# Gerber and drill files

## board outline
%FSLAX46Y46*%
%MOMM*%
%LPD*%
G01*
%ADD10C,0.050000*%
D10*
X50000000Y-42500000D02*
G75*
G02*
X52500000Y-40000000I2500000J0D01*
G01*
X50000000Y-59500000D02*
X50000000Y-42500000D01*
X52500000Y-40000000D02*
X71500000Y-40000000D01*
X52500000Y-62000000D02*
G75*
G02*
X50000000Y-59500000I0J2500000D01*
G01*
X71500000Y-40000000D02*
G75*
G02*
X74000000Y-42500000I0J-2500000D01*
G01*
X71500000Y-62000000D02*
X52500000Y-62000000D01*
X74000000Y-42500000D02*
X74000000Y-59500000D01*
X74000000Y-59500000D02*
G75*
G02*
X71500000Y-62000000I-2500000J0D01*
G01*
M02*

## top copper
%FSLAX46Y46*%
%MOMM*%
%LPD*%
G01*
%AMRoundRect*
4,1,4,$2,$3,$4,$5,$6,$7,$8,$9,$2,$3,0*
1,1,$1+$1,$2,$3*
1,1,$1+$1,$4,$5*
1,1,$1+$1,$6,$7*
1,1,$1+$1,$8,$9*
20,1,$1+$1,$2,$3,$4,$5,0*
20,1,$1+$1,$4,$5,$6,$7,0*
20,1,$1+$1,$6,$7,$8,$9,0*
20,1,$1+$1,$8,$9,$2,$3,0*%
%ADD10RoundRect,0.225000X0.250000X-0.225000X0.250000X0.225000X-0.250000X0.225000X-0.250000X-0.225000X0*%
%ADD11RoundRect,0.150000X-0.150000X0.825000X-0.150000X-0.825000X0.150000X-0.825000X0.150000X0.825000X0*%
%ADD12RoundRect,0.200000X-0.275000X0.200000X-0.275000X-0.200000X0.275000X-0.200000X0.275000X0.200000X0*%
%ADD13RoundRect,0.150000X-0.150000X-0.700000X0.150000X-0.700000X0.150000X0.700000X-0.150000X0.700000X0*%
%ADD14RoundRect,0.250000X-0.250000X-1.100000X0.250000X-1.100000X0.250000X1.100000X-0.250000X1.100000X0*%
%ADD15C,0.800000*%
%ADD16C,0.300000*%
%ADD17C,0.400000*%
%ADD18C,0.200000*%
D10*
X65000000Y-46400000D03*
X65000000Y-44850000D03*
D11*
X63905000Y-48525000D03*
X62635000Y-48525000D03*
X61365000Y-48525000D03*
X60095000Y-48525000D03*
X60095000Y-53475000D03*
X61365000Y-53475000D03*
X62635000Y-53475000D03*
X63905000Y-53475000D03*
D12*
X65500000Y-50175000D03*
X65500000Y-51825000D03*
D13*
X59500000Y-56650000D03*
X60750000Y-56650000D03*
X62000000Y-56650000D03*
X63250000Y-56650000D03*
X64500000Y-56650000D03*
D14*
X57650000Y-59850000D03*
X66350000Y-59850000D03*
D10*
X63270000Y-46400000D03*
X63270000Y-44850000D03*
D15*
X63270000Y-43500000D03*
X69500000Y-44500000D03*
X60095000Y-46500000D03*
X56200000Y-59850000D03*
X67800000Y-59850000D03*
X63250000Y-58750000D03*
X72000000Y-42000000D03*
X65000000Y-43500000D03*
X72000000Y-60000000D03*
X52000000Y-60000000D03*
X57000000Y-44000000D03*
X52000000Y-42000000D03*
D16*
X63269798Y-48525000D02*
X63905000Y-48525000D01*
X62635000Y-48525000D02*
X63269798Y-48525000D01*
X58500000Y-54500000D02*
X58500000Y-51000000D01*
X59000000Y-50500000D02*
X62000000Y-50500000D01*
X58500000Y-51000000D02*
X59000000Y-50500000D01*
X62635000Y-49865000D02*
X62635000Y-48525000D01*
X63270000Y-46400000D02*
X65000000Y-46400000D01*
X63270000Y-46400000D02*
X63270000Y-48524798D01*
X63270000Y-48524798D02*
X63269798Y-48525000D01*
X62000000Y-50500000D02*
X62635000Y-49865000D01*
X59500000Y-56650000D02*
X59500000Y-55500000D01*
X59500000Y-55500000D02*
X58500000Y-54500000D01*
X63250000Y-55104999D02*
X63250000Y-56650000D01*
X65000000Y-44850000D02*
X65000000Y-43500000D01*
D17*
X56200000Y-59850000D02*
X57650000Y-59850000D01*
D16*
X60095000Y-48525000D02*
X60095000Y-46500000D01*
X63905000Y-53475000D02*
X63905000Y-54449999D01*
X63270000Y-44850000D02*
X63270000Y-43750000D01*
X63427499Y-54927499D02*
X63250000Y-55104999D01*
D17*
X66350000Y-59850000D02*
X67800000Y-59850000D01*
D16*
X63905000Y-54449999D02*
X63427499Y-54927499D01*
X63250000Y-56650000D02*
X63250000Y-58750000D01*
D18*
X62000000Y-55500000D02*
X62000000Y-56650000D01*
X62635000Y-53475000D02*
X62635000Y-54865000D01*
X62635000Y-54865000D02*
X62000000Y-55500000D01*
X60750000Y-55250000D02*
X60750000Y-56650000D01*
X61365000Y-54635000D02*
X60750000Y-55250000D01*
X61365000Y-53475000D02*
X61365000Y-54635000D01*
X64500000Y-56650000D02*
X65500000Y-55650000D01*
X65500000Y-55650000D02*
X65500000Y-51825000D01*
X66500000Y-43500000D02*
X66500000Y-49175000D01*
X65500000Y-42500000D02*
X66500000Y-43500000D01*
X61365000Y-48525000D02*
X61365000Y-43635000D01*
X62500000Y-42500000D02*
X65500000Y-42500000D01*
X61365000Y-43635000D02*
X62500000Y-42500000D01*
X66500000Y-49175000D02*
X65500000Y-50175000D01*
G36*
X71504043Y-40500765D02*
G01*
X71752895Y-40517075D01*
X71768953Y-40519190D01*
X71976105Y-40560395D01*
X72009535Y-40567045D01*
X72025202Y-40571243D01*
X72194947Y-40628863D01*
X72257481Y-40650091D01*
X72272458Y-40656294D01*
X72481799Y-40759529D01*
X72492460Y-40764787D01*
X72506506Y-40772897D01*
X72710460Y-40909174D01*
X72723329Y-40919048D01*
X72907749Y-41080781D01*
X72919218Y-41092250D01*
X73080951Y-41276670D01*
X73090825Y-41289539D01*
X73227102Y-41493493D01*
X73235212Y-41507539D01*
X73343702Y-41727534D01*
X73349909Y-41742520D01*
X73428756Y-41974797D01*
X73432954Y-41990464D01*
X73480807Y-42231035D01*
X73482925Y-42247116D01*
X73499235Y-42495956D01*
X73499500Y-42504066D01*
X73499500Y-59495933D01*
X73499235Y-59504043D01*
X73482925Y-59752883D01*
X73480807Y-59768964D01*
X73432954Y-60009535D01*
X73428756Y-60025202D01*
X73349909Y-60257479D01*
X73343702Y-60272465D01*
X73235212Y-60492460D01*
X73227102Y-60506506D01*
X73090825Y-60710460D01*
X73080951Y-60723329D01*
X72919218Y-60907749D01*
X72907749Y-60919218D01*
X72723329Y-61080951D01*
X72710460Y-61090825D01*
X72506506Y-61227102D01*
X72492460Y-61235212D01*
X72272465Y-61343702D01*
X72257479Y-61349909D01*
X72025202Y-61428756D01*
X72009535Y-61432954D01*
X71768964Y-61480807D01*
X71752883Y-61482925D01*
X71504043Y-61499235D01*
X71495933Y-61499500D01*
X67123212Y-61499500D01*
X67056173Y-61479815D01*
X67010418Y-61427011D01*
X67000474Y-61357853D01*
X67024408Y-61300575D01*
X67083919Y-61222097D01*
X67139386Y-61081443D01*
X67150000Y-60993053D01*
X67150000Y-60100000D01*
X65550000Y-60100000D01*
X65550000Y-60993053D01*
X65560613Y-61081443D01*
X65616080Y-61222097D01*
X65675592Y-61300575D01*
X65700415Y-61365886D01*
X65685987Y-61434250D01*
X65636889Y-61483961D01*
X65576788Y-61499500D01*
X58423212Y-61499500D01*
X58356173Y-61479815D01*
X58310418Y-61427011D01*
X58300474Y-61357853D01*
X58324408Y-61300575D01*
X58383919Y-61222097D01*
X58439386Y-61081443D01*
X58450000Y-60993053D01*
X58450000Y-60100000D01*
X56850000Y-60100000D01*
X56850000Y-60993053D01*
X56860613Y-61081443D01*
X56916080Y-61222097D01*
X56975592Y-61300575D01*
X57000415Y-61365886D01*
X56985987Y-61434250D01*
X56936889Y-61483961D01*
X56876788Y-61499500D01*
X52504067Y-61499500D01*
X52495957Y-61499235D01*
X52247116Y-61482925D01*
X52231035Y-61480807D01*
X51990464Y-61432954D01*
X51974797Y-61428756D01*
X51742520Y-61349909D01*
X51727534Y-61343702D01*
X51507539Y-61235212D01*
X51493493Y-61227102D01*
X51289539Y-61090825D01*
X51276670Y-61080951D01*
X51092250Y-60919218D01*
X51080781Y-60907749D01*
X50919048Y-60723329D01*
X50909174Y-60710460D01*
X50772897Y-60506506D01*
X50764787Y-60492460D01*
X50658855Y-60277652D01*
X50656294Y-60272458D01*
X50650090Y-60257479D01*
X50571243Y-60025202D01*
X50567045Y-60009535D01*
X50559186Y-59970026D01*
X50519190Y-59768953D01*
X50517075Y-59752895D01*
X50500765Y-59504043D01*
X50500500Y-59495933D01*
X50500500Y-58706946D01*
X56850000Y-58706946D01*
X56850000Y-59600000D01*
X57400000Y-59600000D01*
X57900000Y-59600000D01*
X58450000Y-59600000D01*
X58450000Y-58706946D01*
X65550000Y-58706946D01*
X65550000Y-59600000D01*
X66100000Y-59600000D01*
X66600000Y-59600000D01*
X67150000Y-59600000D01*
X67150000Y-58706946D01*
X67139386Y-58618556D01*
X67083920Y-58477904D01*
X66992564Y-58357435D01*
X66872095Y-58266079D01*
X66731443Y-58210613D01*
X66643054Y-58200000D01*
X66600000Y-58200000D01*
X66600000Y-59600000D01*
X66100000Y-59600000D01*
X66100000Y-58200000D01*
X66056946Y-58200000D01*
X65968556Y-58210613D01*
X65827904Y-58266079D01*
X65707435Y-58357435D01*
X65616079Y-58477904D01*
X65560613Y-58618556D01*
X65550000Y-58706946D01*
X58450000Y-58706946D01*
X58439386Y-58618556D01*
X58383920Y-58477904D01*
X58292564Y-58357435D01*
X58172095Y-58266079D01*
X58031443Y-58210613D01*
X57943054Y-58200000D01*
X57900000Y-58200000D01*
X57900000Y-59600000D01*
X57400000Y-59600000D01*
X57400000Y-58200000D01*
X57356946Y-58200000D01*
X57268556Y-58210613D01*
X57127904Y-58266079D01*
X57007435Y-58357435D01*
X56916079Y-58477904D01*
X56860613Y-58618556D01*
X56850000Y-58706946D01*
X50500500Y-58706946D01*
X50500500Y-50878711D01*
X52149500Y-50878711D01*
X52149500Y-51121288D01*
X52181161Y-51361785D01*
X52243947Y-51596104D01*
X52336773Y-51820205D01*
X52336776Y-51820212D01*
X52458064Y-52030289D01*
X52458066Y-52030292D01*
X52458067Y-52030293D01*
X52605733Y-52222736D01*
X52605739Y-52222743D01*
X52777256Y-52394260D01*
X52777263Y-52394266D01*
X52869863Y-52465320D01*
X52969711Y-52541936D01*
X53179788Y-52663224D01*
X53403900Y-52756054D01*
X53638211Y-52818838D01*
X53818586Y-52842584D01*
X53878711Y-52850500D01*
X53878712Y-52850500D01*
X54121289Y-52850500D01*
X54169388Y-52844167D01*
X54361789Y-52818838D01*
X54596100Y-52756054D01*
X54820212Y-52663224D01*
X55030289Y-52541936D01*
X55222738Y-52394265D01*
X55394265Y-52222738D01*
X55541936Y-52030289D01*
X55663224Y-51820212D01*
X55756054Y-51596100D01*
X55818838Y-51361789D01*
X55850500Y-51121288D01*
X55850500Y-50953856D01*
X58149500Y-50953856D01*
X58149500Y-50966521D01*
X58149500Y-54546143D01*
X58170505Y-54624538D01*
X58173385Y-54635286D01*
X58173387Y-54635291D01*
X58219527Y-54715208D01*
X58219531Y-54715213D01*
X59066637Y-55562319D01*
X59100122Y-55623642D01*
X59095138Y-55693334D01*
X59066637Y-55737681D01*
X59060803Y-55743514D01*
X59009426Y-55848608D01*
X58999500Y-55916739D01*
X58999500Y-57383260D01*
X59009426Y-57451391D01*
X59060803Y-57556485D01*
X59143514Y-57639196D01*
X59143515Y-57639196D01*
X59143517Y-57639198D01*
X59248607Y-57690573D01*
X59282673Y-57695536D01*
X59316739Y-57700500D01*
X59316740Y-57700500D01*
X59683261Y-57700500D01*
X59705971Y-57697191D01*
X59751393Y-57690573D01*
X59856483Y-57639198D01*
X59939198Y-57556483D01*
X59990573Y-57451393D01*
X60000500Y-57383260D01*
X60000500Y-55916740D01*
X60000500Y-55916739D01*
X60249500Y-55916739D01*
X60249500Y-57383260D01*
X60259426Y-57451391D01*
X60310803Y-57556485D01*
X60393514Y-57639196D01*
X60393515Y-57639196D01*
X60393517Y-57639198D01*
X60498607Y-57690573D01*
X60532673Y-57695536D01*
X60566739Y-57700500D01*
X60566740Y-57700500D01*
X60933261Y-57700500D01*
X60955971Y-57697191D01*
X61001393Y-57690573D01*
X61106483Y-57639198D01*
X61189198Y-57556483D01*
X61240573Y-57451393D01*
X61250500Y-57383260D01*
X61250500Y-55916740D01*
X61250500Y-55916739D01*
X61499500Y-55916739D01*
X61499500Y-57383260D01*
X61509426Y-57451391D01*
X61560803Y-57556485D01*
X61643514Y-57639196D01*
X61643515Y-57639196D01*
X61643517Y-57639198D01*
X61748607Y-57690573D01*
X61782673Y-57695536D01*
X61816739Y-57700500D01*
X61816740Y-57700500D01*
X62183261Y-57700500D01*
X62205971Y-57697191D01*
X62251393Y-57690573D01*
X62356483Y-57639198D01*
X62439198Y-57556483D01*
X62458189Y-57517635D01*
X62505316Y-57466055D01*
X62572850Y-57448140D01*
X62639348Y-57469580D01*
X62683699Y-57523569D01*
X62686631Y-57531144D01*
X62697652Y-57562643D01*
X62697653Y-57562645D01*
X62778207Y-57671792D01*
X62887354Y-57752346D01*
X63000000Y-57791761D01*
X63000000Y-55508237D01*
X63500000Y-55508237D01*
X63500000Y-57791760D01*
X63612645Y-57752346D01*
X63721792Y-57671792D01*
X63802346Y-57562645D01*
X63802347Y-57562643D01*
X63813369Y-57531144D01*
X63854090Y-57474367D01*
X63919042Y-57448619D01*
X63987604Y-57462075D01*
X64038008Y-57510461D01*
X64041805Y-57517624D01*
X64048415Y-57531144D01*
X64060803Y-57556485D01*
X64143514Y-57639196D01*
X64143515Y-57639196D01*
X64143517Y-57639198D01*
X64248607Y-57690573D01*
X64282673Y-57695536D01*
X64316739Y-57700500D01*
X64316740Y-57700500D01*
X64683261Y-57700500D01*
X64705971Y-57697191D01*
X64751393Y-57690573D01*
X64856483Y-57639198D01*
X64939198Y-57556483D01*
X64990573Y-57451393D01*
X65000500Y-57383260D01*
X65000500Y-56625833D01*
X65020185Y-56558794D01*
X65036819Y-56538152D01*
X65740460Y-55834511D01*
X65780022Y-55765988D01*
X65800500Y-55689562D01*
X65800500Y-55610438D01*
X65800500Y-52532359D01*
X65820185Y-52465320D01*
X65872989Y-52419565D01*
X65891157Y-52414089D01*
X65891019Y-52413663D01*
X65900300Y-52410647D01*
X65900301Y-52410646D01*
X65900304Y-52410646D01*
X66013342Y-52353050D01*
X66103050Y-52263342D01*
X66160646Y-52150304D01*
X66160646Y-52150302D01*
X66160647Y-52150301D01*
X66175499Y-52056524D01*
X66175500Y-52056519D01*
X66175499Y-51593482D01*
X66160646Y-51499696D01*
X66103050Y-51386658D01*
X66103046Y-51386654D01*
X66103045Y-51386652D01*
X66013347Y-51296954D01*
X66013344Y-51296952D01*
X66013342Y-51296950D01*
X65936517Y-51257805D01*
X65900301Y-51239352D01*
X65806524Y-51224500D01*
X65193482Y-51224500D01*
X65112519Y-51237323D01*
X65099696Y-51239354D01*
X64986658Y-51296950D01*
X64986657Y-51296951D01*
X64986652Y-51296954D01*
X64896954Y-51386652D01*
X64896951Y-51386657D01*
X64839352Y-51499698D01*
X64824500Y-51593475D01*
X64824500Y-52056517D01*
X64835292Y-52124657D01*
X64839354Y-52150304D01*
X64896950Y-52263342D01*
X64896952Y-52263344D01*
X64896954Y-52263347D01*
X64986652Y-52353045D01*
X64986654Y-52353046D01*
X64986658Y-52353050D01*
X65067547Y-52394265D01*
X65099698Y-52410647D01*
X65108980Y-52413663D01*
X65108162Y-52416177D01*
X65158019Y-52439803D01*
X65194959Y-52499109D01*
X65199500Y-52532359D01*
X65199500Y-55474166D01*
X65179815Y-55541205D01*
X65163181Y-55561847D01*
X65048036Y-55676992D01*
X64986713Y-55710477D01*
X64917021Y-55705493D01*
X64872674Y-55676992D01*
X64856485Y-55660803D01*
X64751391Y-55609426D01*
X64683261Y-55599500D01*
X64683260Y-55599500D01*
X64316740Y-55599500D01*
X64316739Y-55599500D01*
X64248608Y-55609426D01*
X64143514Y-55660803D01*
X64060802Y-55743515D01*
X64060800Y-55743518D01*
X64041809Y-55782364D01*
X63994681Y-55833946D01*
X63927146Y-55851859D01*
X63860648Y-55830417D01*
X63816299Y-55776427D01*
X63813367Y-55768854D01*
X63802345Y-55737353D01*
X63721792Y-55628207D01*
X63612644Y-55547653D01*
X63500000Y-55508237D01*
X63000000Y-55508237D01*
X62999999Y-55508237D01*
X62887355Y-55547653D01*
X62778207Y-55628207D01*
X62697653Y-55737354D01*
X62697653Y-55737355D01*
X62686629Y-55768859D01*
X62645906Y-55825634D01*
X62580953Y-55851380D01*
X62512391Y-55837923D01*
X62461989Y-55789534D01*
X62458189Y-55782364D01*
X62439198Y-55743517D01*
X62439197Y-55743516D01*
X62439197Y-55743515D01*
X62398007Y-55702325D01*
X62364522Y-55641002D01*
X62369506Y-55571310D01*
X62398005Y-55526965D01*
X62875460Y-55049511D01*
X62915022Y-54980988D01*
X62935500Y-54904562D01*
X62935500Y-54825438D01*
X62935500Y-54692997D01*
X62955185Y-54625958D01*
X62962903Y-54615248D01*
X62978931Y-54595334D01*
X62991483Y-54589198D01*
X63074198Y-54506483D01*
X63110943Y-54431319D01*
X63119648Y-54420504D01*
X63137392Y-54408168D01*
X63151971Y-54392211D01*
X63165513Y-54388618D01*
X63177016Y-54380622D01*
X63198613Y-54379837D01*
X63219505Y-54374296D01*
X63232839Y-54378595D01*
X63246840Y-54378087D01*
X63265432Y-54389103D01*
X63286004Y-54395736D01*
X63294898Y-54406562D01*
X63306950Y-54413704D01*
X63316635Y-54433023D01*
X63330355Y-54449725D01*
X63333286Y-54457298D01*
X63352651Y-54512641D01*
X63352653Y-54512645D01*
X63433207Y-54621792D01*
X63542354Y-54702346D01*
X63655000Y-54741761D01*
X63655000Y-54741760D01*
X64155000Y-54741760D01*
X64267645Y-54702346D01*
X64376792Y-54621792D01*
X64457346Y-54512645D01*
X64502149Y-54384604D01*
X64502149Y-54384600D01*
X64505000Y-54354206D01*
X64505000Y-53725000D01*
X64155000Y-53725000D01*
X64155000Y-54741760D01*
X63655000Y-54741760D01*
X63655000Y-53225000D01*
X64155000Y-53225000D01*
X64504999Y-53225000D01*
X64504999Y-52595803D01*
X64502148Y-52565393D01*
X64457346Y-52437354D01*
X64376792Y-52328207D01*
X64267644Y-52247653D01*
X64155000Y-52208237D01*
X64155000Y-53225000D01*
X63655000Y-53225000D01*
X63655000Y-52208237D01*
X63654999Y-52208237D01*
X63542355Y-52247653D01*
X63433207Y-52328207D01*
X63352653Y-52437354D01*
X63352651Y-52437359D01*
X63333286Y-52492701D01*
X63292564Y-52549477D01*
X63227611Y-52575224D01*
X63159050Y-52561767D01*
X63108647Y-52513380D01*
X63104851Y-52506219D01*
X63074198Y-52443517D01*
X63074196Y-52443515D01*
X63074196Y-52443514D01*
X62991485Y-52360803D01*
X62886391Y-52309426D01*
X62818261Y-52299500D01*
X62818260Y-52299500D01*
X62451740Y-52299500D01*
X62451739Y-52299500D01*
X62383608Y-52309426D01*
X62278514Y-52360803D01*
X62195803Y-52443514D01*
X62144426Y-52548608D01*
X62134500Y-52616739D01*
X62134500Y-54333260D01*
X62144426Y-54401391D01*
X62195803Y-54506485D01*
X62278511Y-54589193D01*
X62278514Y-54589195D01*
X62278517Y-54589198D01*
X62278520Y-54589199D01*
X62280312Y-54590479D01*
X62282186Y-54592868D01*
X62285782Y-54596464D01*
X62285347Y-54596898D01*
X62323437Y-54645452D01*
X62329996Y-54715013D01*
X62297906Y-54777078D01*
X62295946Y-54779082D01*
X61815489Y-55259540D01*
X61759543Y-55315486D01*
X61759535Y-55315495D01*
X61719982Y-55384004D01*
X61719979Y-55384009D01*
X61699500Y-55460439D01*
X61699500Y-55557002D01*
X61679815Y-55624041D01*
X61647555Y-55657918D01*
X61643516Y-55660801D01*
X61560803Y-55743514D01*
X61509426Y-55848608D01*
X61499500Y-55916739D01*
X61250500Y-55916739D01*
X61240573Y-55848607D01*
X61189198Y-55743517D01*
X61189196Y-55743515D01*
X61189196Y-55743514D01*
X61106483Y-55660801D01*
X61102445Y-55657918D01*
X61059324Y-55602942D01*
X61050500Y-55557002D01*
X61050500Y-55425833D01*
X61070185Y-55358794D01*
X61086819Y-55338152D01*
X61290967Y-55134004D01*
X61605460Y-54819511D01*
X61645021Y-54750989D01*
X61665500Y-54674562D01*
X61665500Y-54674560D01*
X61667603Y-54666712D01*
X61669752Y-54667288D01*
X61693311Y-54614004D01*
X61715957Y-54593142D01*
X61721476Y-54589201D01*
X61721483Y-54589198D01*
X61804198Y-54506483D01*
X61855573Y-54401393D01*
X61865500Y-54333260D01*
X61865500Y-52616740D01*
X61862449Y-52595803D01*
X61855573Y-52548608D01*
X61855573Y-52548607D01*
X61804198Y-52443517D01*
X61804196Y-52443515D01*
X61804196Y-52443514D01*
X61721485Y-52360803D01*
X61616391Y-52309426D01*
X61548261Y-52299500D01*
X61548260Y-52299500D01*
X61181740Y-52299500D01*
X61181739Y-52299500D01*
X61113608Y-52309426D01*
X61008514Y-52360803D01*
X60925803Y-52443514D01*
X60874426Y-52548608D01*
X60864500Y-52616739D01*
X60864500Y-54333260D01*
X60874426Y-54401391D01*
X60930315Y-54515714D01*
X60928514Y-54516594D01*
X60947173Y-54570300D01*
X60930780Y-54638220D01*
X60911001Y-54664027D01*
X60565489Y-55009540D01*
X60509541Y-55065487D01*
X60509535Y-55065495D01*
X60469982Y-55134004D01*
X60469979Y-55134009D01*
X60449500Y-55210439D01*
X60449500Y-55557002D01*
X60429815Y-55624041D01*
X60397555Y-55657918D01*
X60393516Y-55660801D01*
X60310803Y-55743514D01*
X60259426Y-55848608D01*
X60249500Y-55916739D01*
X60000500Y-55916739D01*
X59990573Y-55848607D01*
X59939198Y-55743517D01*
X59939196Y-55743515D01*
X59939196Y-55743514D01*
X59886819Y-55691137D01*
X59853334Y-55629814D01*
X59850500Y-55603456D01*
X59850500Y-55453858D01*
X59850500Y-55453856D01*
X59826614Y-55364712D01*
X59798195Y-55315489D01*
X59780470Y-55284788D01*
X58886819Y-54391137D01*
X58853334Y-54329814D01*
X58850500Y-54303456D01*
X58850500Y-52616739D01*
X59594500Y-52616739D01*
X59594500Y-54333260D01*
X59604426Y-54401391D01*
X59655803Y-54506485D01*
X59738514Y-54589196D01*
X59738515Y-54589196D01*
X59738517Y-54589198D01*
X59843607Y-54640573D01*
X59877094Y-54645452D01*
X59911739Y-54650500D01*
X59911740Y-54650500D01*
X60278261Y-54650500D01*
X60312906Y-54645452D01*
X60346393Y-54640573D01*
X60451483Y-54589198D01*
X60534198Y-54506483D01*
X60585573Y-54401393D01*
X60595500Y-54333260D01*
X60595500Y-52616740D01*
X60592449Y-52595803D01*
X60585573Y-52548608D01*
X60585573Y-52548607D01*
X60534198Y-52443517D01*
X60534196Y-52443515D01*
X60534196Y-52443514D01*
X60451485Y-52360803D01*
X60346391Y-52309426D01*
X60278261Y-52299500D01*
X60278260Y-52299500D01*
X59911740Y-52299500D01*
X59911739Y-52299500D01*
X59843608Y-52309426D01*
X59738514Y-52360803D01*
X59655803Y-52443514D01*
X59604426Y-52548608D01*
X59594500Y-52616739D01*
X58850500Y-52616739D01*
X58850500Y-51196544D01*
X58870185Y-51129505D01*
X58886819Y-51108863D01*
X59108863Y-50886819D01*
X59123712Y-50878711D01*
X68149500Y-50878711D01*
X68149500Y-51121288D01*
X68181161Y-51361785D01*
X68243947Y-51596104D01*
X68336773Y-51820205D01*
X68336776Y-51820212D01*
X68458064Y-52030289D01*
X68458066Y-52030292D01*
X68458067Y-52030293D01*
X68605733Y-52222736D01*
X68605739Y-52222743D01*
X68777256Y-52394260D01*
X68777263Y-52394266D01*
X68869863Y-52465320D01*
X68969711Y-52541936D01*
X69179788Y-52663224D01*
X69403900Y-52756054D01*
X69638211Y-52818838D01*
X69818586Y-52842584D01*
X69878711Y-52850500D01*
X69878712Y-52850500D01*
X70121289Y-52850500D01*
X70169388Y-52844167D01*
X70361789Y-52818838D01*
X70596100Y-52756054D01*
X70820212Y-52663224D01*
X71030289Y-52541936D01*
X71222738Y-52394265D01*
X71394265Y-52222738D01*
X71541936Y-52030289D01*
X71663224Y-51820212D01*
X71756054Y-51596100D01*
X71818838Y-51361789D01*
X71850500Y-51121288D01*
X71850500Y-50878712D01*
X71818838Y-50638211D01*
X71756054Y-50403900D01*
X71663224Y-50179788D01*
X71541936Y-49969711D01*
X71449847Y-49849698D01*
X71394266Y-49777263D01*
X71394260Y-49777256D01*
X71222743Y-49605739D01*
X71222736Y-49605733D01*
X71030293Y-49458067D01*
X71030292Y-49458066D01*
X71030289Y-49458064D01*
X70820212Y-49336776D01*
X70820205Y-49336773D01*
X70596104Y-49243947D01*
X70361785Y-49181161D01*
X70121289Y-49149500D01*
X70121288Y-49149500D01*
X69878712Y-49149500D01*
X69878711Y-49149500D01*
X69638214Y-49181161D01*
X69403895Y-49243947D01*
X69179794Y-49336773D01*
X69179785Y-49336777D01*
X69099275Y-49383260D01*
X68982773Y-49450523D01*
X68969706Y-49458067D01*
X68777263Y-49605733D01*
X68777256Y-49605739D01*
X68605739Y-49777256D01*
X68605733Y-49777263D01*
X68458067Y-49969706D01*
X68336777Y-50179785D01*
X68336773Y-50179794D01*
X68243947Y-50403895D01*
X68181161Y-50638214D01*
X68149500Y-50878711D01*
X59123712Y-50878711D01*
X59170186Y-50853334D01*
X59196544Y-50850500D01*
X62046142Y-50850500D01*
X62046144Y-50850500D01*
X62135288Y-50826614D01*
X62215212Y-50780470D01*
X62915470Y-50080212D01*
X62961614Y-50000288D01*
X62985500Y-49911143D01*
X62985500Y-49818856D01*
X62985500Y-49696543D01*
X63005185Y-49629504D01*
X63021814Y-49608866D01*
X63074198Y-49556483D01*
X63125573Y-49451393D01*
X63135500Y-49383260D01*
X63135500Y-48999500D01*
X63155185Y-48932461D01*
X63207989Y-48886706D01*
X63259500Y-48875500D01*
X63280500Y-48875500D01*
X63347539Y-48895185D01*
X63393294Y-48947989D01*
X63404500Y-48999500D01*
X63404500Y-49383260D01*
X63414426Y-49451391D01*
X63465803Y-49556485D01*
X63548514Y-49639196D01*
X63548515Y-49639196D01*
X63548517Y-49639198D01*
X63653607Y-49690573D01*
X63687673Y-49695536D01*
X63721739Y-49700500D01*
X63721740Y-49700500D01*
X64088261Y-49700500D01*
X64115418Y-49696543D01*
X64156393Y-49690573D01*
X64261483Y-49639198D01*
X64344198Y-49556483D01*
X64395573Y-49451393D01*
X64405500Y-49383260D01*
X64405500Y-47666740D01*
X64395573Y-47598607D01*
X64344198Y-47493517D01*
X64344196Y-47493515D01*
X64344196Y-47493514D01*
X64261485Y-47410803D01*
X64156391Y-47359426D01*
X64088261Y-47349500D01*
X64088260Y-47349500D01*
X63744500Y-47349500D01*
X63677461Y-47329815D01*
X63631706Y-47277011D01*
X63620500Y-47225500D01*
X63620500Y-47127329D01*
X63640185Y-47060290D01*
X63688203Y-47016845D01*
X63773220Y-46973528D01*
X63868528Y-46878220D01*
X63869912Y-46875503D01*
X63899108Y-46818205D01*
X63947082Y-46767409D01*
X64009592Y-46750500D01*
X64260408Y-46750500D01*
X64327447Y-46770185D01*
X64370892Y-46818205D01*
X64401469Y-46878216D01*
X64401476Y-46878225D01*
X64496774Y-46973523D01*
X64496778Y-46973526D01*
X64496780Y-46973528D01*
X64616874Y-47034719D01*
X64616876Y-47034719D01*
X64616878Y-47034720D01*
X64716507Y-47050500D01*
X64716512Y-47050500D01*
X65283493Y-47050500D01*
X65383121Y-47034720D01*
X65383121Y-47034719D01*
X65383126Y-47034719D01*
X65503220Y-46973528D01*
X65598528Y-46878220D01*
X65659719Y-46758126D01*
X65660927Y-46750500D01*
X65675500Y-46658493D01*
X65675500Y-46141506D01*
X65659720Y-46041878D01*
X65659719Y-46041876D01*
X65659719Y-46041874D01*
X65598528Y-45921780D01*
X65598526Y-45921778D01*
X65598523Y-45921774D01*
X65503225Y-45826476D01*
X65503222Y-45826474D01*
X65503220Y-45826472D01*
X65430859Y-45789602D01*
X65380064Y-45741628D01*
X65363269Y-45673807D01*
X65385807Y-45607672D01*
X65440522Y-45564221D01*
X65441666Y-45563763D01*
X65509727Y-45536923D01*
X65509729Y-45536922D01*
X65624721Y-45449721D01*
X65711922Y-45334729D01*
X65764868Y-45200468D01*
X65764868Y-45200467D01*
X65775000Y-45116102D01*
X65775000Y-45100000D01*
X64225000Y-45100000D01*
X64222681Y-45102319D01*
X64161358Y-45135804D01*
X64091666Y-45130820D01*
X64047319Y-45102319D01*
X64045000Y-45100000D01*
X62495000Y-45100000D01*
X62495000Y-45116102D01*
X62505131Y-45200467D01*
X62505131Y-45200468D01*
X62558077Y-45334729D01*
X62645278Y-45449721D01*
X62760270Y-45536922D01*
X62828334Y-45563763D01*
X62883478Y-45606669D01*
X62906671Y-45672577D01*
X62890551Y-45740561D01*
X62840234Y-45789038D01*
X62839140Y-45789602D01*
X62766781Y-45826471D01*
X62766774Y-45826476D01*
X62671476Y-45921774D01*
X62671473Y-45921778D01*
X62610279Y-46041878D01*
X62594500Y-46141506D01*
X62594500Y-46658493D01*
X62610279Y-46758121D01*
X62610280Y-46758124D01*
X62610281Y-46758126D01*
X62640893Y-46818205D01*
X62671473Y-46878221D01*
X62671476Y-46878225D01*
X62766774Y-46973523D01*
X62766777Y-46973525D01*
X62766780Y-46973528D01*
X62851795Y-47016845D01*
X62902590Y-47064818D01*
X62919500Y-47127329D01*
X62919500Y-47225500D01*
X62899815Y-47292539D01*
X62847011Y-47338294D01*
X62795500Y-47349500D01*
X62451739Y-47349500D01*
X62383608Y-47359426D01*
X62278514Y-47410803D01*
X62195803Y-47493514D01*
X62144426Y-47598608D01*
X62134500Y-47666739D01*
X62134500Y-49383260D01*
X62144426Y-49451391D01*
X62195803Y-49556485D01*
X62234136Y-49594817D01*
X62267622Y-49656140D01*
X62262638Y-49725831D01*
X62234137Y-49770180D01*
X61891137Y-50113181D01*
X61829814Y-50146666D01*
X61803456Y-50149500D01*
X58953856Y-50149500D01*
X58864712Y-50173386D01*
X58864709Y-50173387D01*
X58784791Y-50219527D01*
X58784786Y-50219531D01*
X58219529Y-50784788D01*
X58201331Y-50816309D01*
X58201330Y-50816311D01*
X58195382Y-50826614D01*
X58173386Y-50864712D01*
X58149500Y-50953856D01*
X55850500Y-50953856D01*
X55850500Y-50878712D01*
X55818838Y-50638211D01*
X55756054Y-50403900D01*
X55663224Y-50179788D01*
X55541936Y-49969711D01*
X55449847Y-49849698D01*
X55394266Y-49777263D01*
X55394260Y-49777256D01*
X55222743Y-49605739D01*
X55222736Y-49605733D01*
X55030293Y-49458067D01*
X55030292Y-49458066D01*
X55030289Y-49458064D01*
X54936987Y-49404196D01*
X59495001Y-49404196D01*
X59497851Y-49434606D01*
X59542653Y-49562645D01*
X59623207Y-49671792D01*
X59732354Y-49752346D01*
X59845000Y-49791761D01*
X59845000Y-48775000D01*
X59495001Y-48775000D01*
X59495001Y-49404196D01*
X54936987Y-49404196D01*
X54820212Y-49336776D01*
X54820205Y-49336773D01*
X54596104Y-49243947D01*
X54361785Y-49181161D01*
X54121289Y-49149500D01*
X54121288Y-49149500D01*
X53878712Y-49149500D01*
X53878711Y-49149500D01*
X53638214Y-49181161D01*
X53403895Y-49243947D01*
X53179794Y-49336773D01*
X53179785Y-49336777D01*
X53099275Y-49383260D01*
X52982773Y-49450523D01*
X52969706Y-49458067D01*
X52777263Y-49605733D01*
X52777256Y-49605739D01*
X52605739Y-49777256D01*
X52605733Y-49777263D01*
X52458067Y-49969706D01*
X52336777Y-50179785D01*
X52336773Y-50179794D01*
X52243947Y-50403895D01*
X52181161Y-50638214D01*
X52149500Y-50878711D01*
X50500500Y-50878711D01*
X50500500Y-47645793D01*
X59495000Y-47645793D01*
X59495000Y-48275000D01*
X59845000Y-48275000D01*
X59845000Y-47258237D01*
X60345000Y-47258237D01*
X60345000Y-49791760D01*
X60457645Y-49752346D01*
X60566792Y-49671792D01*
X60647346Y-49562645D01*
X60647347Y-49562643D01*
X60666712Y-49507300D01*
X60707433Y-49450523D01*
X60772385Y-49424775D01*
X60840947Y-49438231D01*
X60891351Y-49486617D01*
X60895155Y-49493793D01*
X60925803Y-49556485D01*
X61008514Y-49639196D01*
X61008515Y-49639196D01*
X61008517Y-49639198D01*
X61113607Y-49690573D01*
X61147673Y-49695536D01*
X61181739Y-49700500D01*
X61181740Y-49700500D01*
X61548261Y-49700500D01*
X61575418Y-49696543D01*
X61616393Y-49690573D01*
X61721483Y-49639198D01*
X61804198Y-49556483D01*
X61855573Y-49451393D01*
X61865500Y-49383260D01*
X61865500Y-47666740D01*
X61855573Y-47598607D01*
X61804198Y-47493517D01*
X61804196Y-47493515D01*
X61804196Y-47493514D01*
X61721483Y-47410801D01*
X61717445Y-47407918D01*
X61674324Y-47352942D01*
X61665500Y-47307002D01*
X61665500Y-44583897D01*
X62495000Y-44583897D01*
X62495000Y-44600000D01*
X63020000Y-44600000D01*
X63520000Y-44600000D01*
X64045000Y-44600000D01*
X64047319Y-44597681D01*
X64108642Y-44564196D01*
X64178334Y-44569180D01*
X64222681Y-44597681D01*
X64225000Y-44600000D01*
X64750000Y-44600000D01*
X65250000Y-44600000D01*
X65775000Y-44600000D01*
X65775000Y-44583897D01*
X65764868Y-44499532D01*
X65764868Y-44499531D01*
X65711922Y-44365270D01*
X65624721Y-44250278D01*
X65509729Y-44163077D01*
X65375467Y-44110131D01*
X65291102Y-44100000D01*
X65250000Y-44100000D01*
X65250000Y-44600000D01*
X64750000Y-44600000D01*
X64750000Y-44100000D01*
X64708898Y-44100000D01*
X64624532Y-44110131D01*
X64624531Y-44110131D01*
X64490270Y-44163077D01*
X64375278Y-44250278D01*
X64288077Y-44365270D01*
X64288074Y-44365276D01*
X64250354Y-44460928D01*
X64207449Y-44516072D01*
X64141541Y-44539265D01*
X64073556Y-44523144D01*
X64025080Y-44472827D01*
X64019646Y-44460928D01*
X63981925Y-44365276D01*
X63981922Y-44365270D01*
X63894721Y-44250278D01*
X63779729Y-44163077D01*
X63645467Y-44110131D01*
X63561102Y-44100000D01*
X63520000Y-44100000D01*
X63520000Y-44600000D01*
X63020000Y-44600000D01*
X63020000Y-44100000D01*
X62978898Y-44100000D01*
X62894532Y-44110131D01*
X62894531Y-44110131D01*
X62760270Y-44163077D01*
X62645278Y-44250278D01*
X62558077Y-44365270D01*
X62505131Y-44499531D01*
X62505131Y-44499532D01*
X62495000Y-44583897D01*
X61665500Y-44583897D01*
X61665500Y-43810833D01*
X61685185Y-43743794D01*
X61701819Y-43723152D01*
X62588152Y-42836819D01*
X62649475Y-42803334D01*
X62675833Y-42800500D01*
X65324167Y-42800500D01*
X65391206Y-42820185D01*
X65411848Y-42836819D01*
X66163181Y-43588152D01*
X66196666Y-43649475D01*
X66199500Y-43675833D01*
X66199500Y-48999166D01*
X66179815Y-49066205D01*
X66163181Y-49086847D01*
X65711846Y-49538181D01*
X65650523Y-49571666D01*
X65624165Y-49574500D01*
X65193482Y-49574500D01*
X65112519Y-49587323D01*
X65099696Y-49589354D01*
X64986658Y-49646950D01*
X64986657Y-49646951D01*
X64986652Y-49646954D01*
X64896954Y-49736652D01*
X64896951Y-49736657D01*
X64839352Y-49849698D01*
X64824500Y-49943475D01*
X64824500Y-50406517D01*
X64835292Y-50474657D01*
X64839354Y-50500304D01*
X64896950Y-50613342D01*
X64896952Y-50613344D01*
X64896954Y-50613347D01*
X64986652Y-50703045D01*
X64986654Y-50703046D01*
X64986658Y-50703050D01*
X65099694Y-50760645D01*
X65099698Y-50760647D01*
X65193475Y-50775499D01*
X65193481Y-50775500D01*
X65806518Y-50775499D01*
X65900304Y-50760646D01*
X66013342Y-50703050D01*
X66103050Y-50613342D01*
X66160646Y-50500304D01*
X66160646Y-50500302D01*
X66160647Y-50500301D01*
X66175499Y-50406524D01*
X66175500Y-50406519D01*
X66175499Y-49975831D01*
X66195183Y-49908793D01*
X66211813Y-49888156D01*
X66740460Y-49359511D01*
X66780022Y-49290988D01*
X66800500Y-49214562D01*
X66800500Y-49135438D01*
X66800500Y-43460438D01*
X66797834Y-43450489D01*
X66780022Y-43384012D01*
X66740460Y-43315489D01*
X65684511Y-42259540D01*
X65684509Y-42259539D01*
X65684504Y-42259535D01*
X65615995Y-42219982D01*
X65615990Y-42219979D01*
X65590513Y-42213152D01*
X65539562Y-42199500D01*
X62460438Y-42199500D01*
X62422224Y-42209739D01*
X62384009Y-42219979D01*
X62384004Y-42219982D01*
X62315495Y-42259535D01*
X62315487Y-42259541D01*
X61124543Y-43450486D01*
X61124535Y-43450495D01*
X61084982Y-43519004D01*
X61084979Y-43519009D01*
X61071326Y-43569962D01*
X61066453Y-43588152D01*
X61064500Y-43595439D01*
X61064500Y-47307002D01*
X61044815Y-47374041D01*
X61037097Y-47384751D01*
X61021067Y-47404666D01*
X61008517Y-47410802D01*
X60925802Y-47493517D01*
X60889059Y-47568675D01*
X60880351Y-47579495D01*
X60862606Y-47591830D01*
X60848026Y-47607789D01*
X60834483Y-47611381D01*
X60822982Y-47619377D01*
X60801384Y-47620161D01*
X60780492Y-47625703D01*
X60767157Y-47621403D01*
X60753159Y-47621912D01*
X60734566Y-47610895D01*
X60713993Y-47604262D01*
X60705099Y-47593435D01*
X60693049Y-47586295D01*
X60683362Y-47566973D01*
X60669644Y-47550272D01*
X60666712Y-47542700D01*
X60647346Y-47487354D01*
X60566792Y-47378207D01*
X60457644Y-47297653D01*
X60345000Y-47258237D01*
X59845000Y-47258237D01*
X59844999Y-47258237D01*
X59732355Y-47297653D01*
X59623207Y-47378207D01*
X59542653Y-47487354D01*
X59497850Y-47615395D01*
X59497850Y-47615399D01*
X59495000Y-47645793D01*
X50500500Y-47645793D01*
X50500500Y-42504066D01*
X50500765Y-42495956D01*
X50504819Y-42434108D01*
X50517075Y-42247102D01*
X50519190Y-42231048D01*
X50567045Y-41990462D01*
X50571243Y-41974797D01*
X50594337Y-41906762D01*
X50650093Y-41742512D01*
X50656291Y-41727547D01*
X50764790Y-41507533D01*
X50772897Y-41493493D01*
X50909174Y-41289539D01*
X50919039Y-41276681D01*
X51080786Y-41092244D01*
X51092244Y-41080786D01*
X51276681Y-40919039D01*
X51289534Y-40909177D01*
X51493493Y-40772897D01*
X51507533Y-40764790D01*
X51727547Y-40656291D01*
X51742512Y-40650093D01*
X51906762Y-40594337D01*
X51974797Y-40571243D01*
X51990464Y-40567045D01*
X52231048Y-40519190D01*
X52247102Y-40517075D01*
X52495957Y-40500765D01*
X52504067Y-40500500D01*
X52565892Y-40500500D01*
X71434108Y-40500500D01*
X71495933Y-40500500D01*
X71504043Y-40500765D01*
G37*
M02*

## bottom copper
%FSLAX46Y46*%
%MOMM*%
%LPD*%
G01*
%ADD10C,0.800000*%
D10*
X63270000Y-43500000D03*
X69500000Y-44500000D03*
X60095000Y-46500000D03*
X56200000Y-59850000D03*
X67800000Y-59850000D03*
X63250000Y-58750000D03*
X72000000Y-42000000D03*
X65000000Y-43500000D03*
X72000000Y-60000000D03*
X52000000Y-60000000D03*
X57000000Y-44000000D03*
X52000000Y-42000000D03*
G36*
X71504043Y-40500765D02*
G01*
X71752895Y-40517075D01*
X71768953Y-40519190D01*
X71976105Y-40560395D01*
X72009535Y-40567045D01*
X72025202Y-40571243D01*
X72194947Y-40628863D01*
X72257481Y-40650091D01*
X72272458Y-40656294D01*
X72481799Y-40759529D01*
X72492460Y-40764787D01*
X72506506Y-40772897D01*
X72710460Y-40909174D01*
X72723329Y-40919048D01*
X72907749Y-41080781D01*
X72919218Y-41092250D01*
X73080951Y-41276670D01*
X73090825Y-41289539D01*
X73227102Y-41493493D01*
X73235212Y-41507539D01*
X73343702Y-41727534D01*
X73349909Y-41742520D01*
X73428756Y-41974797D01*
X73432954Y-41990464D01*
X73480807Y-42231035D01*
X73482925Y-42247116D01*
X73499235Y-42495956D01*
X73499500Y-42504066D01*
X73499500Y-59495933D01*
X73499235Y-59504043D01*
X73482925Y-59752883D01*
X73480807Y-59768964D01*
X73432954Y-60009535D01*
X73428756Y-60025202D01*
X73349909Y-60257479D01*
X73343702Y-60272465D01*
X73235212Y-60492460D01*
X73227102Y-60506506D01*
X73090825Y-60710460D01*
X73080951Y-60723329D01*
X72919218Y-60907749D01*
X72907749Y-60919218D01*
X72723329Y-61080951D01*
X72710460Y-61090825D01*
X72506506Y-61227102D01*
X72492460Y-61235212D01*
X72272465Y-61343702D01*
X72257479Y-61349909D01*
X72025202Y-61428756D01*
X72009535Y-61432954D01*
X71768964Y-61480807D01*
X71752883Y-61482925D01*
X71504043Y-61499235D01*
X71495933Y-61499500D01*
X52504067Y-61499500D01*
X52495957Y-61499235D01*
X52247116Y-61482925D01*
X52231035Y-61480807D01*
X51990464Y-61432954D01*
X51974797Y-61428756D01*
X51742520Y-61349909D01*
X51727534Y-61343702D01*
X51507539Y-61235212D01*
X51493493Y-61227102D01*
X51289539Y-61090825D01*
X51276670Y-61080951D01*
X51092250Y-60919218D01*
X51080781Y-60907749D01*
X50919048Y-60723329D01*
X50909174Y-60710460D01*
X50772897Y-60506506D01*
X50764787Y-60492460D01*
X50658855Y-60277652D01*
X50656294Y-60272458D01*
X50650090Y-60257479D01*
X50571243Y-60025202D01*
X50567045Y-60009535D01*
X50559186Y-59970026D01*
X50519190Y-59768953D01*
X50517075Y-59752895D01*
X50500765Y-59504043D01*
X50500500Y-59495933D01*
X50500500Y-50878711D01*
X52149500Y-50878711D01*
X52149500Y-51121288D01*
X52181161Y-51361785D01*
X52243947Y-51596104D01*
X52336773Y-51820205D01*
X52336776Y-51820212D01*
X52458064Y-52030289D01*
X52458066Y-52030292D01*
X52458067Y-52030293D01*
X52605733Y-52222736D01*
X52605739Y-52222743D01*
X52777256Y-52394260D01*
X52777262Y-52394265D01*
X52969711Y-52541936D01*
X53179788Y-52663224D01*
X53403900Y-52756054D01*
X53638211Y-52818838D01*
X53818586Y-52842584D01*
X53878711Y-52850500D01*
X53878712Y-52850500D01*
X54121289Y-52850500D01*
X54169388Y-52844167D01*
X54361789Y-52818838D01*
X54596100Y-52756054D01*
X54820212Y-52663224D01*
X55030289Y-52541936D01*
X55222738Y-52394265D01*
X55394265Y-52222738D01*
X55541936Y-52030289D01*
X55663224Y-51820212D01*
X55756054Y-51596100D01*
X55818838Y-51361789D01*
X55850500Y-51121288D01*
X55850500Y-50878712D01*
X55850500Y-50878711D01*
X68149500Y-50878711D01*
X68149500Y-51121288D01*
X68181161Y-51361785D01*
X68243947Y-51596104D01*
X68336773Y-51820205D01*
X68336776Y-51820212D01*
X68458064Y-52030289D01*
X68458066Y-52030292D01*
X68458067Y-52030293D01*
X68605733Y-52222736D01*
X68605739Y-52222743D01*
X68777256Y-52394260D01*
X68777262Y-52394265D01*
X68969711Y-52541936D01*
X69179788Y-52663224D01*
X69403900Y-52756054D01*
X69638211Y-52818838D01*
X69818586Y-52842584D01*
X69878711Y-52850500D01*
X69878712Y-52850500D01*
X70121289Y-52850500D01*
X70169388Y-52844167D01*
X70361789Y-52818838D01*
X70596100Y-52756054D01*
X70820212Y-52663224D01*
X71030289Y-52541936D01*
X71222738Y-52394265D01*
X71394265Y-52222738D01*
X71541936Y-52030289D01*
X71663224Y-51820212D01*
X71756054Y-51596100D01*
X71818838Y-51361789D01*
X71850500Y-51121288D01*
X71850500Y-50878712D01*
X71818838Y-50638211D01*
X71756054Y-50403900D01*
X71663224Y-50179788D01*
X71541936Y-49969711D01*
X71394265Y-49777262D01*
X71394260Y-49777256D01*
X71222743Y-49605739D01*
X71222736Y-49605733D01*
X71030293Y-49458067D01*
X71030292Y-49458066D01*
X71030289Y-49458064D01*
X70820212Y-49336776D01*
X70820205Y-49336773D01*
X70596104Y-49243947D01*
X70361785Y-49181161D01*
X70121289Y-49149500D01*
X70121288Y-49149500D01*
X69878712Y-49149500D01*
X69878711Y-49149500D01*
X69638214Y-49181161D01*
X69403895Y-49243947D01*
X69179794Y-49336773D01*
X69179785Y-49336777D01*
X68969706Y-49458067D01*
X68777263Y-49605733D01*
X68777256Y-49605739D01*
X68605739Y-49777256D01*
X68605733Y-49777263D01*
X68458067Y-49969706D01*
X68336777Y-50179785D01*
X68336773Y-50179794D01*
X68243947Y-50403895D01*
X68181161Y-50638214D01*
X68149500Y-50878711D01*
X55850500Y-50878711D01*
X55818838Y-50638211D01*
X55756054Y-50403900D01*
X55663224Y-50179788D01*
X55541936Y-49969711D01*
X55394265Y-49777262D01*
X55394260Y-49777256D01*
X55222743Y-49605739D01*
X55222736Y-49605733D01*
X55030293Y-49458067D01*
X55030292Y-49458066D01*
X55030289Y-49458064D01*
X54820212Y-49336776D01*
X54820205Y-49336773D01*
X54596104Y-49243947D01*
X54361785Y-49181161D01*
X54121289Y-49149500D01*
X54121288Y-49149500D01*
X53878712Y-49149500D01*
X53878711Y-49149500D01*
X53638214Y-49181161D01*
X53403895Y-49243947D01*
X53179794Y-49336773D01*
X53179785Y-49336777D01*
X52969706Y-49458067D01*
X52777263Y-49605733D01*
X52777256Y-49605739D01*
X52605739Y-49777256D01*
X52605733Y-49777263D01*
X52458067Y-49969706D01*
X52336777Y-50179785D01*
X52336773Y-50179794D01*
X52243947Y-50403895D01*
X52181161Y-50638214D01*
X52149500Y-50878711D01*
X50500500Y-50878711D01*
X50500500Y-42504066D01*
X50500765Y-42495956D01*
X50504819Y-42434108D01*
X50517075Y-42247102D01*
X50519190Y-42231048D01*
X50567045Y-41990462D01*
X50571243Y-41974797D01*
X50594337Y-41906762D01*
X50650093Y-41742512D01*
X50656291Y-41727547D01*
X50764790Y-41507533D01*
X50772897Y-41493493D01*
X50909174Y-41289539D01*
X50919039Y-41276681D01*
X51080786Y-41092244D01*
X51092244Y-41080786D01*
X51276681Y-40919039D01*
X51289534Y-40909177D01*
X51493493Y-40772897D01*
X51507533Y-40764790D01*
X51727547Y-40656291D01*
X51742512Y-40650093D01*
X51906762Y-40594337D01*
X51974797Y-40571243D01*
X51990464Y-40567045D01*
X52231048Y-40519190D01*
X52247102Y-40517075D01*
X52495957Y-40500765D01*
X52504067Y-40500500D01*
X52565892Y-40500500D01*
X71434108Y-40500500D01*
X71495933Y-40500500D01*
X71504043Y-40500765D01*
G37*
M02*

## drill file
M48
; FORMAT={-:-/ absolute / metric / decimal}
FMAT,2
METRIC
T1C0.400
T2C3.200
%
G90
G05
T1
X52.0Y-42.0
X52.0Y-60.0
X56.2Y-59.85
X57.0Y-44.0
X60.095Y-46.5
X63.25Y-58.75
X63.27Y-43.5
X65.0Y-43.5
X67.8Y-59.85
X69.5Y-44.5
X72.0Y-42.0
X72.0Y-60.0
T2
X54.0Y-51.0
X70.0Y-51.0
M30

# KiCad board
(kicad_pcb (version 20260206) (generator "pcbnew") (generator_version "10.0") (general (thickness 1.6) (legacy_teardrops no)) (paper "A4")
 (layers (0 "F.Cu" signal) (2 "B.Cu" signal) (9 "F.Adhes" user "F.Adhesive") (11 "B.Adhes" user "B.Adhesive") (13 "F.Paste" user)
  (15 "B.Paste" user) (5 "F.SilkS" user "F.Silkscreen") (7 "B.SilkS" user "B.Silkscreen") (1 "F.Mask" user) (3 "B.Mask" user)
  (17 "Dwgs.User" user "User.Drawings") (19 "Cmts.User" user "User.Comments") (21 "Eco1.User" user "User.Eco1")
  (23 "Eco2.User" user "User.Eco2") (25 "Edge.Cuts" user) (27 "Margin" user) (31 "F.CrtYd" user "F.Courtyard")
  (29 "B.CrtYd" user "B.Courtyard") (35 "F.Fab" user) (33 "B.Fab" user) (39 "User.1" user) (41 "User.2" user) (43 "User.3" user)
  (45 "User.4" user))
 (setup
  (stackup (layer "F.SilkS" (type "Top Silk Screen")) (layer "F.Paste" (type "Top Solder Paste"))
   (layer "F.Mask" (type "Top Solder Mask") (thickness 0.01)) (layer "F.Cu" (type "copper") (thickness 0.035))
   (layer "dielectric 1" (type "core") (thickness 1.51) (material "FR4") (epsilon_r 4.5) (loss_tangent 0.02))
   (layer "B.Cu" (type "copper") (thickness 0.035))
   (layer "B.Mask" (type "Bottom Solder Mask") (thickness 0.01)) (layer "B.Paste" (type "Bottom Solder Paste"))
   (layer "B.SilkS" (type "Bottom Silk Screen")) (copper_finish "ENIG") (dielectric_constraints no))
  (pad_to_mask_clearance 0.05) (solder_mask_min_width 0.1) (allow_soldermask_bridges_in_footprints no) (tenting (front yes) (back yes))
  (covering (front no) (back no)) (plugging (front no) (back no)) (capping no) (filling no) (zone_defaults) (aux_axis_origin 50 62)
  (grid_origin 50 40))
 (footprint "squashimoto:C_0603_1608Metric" (layer "F.Cu") (at 65 45.625 90)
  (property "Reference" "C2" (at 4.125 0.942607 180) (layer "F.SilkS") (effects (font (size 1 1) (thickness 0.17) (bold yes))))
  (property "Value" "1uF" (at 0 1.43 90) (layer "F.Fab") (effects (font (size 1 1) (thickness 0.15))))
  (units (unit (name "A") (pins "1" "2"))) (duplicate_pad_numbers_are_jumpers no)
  (pad "1" smd roundrect (at -0.775 0 90) (size 0.9 0.95) (layers "F.Cu" "F.Mask" "F.Paste") (roundrect_rratio 0.25) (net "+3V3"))
  (pad "2" smd roundrect (at 0.775 0 90) (size 0.9 0.95) (layers "F.Cu" "F.Mask" "F.Paste") (roundrect_rratio 0.25) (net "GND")))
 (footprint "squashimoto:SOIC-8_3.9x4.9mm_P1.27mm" (layer "F.Cu") (at 62 51 -90)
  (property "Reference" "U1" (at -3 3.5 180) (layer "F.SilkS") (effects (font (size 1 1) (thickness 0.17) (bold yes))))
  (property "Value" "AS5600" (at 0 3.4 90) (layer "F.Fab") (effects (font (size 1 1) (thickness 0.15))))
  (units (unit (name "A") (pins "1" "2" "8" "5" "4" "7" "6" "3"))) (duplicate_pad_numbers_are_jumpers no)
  (pad "1" smd roundrect (at -2.475 -1.905 270) (size 1.95 0.6) (layers "F.Cu" "F.Mask" "F.Paste") (roundrect_rratio 0.25) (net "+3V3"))
  (pad "2" smd roundrect (at -2.475 -0.635 270) (size 1.95 0.6) (layers "F.Cu" "F.Mask" "F.Paste") (roundrect_rratio 0.25) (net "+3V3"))
  (pad "3" smd roundrect (at -2.475 0.635 270) (size 1.95 0.6) (layers "F.Cu" "F.Mask" "F.Paste") (roundrect_rratio 0.25)
   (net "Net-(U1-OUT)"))
  (pad "4" smd roundrect (at -2.475 1.905 270) (size 1.95 0.6) (layers "F.Cu" "F.Mask" "F.Paste") (roundrect_rratio 0.25) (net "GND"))
  (pad "5" smd roundrect (at 2.475 1.905 270) (size 1.95 0.6) (layers "F.Cu" "F.Mask" "F.Paste") (roundrect_rratio 0.25)
   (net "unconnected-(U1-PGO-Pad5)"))
  (pad "6" smd roundrect (at 2.475 0.635 270) (size 1.95 0.6) (layers "F.Cu" "F.Mask" "F.Paste") (roundrect_rratio 0.25) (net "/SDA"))
  (pad "7" smd roundrect (at 2.475 -0.635 270) (size 1.95 0.6) (layers "F.Cu" "F.Mask" "F.Paste") (roundrect_rratio 0.25) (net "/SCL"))
  (pad "8" smd roundrect (at 2.475 -1.905 270) (size 1.95 0.6) (layers "F.Cu" "F.Mask" "F.Paste") (roundrect_rratio 0.25) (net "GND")))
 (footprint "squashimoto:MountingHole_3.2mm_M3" (layer "F.Cu") (at 54 51)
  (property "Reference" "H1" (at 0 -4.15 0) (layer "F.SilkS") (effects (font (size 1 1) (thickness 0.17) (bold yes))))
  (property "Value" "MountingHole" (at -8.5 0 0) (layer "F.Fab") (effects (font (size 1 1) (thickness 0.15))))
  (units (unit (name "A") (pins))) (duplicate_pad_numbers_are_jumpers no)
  (pad "" np_thru_hole circle (at 0 0) (size 3.2 3.2) (drill 3.2) (layers "*.Cu" "*.Mask")))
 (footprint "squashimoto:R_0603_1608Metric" (layer "F.Cu") (at 65.5 51 -90)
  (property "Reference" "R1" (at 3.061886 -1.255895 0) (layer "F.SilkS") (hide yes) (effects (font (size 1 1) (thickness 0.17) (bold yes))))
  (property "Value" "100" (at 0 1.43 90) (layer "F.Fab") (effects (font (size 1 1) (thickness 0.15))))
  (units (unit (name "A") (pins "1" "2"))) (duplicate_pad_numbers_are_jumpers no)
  (pad "1" smd roundrect (at -0.825 0 270) (size 0.8 0.95) (layers "F.Cu" "F.Mask" "F.Paste") (roundrect_rratio 0.25) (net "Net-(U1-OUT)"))
  (pad "2" smd roundrect (at 0.825 0 270) (size 0.8 0.95) (layers "F.Cu" "F.Mask" "F.Paste") (roundrect_rratio 0.25) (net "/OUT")))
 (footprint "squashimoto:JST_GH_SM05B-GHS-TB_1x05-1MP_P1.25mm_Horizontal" (layer "F.Cu") (at 62 58.5)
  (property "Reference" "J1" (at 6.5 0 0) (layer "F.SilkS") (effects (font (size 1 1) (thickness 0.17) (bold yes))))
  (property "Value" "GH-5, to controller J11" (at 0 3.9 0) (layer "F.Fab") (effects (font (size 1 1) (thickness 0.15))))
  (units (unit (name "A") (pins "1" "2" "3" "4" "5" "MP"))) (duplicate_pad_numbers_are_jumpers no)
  (pad "1" smd roundrect (at -2.5 -1.85) (size 0.6 1.7) (layers "F.Cu" "F.Mask" "F.Paste") (roundrect_rratio 0.25) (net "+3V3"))
  (pad "2" smd roundrect (at -1.25 -1.85) (size 0.6 1.7) (layers "F.Cu" "F.Mask" "F.Paste") (roundrect_rratio 0.25) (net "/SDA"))
  (pad "3" smd roundrect (at 0 -1.85) (size 0.6 1.7) (layers "F.Cu" "F.Mask" "F.Paste") (roundrect_rratio 0.25) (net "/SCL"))
  (pad "4" smd roundrect (at 1.25 -1.85) (size 0.6 1.7) (layers "F.Cu" "F.Mask" "F.Paste") (roundrect_rratio 0.25) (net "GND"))
  (pad "5" smd roundrect (at 2.5 -1.85) (size 0.6 1.7) (layers "F.Cu" "F.Mask" "F.Paste") (roundrect_rratio 0.25) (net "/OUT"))
  (pad "MP" smd roundrect (at -4.35 1.35) (size 1 2.7) (layers "F.Cu" "F.Mask" "F.Paste") (roundrect_rratio 0.25) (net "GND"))
  (pad "MP" smd roundrect (at 4.35 1.35) (size 1 2.7) (layers "F.Cu" "F.Mask" "F.Paste") (roundrect_rratio 0.25) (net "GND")))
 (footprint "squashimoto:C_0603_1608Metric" (layer "F.Cu") (at 63.27 45.625 90)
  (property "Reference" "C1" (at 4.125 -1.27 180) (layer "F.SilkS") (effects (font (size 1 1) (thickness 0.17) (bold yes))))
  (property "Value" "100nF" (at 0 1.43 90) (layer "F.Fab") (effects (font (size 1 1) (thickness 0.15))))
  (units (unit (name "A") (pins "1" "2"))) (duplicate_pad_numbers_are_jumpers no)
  (pad "1" smd roundrect (at -0.775 0 90) (size 0.9 0.95) (layers "F.Cu" "F.Mask" "F.Paste") (roundrect_rratio 0.25) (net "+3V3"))
  (pad "2" smd roundrect (at 0.775 0 90) (size 0.9 0.95) (layers "F.Cu" "F.Mask" "F.Paste") (roundrect_rratio 0.25) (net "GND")))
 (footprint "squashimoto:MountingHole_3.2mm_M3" (layer "F.Cu") (at 70 51)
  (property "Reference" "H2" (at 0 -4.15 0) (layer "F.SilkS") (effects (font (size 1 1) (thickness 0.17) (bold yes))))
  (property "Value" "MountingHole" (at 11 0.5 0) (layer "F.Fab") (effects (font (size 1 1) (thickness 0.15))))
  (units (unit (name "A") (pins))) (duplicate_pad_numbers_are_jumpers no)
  (pad "" np_thru_hole circle (at 0 0) (size 3.2 3.2) (drill 3.2) (layers "*.Cu" "*.Mask")))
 (gr_arc (start 50 42.5) (mid 50.732233 40.732233) (end 52.5 40) (stroke (width 0.05) (type default)) (layer "Edge.Cuts"))
 (gr_line (start 50 59.5) (end 50 42.5) (stroke (width 0.05) (type default)) (layer "Edge.Cuts"))
 (gr_line (start 52.5 40) (end 71.5 40) (stroke (width 0.05) (type default)) (layer "Edge.Cuts"))
 (gr_arc (start 52.5 62) (mid 50.732233 61.267767) (end 50 59.5) (stroke (width 0.05) (type default)) (layer "Edge.Cuts"))
 (gr_arc (start 71.5 40) (mid 73.267767 40.732233) (end 74 42.5) (stroke (width 0.05) (type default)) (layer "Edge.Cuts"))
 (gr_line (start 71.5 62) (end 52.5 62) (stroke (width 0.05) (type default)) (layer "Edge.Cuts"))
 (gr_line (start 74 42.5) (end 74 59.5) (stroke (width 0.05) (type default)) (layer "Edge.Cuts"))
 (gr_arc (start 74 59.5) (mid 73.267767 61.267767) (end 71.5 62) (stroke (width 0.05) (type default)) (layer "Edge.Cuts"))
 (segment (start 63.269798 48.525) (end 63.905 48.525) (width 0.3) (layer "F.Cu") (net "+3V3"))
 (segment (start 62.635 48.525) (end 63.269798 48.525) (width 0.3) (layer "F.Cu") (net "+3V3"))
 (segment (start 58.5 54.5) (end 58.5 51) (width 0.3) (layer "F.Cu") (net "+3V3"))
 (segment (start 59 50.5) (end 62 50.5) (width 0.3) (layer "F.Cu") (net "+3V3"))
 (segment (start 58.5 51) (end 59 50.5) (width 0.3) (layer "F.Cu") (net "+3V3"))
 (segment (start 62.635 49.865) (end 62.635 48.525) (width 0.3) (layer "F.Cu") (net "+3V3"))
 (segment (start 63.27 46.4) (end 65 46.4) (width 0.3) (layer "F.Cu") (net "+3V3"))
 (segment (start 63.27 46.4) (end 63.27 48.524798) (width 0.3) (layer "F.Cu") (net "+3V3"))
 (segment (start 63.27 48.524798) (end 63.269798 48.525) (width 0.3) (layer "F.Cu") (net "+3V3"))
 (segment (start 62 50.5) (end 62.635 49.865) (width 0.3) (layer "F.Cu") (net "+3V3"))
 (segment (start 59.5 56.65) (end 59.5 55.5) (width 0.3) (layer "F.Cu") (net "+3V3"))
 (segment (start 59.5 55.5) (end 58.5 54.5) (width 0.3) (layer "F.Cu") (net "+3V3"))
 (segment (start 63.25 55.104999) (end 63.25 56.65) (width 0.3) (layer "F.Cu") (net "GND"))
 (segment (start 65 44.85) (end 65 43.5) (width 0.3) (layer "F.Cu") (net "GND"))
 (segment (start 56.2 59.85) (end 57.65 59.85) (width 0.4) (layer "F.Cu") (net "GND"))
 (segment (start 60.095 48.525) (end 60.095 46.5) (width 0.3) (layer "F.Cu") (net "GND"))
 (segment (start 63.905 53.475) (end 63.905 54.449999) (width 0.3) (layer "F.Cu") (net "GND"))
 (segment (start 63.27 44.85) (end 63.27 43.75) (width 0.3) (layer "F.Cu") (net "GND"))
 (segment (start 63.427499 54.927499) (end 63.25 55.104999) (width 0.3) (layer "F.Cu") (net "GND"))
 (segment (start 66.35 59.85) (end 67.8 59.85) (width 0.4) (layer "F.Cu") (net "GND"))
 (segment (start 63.905 54.449999) (end 63.427499 54.927499) (width 0.3) (layer "F.Cu") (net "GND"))
 (segment (start 63.25 56.65) (end 63.25 58.75) (width 0.3) (layer "F.Cu") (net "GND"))
 (via (at 63.27 43.5) (size 0.8) (drill 0.4) (layers "F.Cu" "B.Cu") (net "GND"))
 (via (at 69.5 44.5) (size 0.8) (drill 0.4) (layers "F.Cu" "B.Cu") (free yes) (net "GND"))
 (via (at 60.095 46.5) (size 0.8) (drill 0.4) (layers "F.Cu" "B.Cu") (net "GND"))
 (via (at 56.2 59.85) (size 0.8) (drill 0.4) (layers "F.Cu" "B.Cu") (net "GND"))
 (via (at 67.8 59.85) (size 0.8) (drill 0.4) (layers "F.Cu" "B.Cu") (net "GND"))
 (via (at 63.25 58.75) (size 0.8) (drill 0.4) (layers "F.Cu" "B.Cu") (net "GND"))
 (via (at 72 42) (size 0.8) (drill 0.4) (layers "F.Cu" "B.Cu") (free yes) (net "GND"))
 (via (at 65 43.5) (size 0.8) (drill 0.4) (layers "F.Cu" "B.Cu") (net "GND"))
 (via (at 72 60) (size 0.8) (drill 0.4) (layers "F.Cu" "B.Cu") (free yes) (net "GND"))
 (via (at 52 60) (size 0.8) (drill 0.4) (layers "F.Cu" "B.Cu") (free yes) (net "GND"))
 (via (at 57 44) (size 0.8) (drill 0.4) (layers "F.Cu" "B.Cu") (free yes) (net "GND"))
 (via (at 52 42) (size 0.8) (drill 0.4) (layers "F.Cu" "B.Cu") (free yes) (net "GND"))
 (segment (start 62 55.5) (end 62 56.65) (width 0.2) (layer "F.Cu") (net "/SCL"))
 (segment (start 62.635 53.475) (end 62.635 54.865) (width 0.2) (layer "F.Cu") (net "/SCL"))
 (segment (start 62.635 54.865) (end 62 55.5) (width 0.2) (layer "F.Cu") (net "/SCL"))
 (segment (start 60.75 55.25) (end 60.75 56.65) (width 0.2) (layer "F.Cu") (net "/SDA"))
 (segment (start 61.365 54.635) (end 60.75 55.25) (width 0.2) (layer "F.Cu") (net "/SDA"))
 (segment (start 61.365 53.475) (end 61.365 54.635) (width 0.2) (layer "F.Cu") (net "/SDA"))
 (segment (start 64.5 56.65) (end 65.5 55.65) (width 0.2) (layer "F.Cu") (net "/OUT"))
 (segment (start 65.5 55.65) (end 65.5 51.825) (width 0.2) (layer "F.Cu") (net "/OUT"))
 (segment (start 66.5 43.5) (end 66.5 49.175) (width 0.2) (layer "F.Cu") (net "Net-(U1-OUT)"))
 (segment (start 65.5 42.5) (end 66.5 43.5) (width 0.2) (layer "F.Cu") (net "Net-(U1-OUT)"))
 (segment (start 61.365 48.525) (end 61.365 43.635) (width 0.2) (layer "F.Cu") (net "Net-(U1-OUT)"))
 (segment (start 62.5 42.5) (end 65.5 42.5) (width 0.2) (layer "F.Cu") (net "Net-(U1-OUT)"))
 (segment (start 61.365 43.635) (end 62.5 42.5) (width 0.2) (layer "F.Cu") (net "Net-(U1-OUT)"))
 (segment (start 66.5 49.175) (end 65.5 50.175) (width 0.2) (layer "F.Cu") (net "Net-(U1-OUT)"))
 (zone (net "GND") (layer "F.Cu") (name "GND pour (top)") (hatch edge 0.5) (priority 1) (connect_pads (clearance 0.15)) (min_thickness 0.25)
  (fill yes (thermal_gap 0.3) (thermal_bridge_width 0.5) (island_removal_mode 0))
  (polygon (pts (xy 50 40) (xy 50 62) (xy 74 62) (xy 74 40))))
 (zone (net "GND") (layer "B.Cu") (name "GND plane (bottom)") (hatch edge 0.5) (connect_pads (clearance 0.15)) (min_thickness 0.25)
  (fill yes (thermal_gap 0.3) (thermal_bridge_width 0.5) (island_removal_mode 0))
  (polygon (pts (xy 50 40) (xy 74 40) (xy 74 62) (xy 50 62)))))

